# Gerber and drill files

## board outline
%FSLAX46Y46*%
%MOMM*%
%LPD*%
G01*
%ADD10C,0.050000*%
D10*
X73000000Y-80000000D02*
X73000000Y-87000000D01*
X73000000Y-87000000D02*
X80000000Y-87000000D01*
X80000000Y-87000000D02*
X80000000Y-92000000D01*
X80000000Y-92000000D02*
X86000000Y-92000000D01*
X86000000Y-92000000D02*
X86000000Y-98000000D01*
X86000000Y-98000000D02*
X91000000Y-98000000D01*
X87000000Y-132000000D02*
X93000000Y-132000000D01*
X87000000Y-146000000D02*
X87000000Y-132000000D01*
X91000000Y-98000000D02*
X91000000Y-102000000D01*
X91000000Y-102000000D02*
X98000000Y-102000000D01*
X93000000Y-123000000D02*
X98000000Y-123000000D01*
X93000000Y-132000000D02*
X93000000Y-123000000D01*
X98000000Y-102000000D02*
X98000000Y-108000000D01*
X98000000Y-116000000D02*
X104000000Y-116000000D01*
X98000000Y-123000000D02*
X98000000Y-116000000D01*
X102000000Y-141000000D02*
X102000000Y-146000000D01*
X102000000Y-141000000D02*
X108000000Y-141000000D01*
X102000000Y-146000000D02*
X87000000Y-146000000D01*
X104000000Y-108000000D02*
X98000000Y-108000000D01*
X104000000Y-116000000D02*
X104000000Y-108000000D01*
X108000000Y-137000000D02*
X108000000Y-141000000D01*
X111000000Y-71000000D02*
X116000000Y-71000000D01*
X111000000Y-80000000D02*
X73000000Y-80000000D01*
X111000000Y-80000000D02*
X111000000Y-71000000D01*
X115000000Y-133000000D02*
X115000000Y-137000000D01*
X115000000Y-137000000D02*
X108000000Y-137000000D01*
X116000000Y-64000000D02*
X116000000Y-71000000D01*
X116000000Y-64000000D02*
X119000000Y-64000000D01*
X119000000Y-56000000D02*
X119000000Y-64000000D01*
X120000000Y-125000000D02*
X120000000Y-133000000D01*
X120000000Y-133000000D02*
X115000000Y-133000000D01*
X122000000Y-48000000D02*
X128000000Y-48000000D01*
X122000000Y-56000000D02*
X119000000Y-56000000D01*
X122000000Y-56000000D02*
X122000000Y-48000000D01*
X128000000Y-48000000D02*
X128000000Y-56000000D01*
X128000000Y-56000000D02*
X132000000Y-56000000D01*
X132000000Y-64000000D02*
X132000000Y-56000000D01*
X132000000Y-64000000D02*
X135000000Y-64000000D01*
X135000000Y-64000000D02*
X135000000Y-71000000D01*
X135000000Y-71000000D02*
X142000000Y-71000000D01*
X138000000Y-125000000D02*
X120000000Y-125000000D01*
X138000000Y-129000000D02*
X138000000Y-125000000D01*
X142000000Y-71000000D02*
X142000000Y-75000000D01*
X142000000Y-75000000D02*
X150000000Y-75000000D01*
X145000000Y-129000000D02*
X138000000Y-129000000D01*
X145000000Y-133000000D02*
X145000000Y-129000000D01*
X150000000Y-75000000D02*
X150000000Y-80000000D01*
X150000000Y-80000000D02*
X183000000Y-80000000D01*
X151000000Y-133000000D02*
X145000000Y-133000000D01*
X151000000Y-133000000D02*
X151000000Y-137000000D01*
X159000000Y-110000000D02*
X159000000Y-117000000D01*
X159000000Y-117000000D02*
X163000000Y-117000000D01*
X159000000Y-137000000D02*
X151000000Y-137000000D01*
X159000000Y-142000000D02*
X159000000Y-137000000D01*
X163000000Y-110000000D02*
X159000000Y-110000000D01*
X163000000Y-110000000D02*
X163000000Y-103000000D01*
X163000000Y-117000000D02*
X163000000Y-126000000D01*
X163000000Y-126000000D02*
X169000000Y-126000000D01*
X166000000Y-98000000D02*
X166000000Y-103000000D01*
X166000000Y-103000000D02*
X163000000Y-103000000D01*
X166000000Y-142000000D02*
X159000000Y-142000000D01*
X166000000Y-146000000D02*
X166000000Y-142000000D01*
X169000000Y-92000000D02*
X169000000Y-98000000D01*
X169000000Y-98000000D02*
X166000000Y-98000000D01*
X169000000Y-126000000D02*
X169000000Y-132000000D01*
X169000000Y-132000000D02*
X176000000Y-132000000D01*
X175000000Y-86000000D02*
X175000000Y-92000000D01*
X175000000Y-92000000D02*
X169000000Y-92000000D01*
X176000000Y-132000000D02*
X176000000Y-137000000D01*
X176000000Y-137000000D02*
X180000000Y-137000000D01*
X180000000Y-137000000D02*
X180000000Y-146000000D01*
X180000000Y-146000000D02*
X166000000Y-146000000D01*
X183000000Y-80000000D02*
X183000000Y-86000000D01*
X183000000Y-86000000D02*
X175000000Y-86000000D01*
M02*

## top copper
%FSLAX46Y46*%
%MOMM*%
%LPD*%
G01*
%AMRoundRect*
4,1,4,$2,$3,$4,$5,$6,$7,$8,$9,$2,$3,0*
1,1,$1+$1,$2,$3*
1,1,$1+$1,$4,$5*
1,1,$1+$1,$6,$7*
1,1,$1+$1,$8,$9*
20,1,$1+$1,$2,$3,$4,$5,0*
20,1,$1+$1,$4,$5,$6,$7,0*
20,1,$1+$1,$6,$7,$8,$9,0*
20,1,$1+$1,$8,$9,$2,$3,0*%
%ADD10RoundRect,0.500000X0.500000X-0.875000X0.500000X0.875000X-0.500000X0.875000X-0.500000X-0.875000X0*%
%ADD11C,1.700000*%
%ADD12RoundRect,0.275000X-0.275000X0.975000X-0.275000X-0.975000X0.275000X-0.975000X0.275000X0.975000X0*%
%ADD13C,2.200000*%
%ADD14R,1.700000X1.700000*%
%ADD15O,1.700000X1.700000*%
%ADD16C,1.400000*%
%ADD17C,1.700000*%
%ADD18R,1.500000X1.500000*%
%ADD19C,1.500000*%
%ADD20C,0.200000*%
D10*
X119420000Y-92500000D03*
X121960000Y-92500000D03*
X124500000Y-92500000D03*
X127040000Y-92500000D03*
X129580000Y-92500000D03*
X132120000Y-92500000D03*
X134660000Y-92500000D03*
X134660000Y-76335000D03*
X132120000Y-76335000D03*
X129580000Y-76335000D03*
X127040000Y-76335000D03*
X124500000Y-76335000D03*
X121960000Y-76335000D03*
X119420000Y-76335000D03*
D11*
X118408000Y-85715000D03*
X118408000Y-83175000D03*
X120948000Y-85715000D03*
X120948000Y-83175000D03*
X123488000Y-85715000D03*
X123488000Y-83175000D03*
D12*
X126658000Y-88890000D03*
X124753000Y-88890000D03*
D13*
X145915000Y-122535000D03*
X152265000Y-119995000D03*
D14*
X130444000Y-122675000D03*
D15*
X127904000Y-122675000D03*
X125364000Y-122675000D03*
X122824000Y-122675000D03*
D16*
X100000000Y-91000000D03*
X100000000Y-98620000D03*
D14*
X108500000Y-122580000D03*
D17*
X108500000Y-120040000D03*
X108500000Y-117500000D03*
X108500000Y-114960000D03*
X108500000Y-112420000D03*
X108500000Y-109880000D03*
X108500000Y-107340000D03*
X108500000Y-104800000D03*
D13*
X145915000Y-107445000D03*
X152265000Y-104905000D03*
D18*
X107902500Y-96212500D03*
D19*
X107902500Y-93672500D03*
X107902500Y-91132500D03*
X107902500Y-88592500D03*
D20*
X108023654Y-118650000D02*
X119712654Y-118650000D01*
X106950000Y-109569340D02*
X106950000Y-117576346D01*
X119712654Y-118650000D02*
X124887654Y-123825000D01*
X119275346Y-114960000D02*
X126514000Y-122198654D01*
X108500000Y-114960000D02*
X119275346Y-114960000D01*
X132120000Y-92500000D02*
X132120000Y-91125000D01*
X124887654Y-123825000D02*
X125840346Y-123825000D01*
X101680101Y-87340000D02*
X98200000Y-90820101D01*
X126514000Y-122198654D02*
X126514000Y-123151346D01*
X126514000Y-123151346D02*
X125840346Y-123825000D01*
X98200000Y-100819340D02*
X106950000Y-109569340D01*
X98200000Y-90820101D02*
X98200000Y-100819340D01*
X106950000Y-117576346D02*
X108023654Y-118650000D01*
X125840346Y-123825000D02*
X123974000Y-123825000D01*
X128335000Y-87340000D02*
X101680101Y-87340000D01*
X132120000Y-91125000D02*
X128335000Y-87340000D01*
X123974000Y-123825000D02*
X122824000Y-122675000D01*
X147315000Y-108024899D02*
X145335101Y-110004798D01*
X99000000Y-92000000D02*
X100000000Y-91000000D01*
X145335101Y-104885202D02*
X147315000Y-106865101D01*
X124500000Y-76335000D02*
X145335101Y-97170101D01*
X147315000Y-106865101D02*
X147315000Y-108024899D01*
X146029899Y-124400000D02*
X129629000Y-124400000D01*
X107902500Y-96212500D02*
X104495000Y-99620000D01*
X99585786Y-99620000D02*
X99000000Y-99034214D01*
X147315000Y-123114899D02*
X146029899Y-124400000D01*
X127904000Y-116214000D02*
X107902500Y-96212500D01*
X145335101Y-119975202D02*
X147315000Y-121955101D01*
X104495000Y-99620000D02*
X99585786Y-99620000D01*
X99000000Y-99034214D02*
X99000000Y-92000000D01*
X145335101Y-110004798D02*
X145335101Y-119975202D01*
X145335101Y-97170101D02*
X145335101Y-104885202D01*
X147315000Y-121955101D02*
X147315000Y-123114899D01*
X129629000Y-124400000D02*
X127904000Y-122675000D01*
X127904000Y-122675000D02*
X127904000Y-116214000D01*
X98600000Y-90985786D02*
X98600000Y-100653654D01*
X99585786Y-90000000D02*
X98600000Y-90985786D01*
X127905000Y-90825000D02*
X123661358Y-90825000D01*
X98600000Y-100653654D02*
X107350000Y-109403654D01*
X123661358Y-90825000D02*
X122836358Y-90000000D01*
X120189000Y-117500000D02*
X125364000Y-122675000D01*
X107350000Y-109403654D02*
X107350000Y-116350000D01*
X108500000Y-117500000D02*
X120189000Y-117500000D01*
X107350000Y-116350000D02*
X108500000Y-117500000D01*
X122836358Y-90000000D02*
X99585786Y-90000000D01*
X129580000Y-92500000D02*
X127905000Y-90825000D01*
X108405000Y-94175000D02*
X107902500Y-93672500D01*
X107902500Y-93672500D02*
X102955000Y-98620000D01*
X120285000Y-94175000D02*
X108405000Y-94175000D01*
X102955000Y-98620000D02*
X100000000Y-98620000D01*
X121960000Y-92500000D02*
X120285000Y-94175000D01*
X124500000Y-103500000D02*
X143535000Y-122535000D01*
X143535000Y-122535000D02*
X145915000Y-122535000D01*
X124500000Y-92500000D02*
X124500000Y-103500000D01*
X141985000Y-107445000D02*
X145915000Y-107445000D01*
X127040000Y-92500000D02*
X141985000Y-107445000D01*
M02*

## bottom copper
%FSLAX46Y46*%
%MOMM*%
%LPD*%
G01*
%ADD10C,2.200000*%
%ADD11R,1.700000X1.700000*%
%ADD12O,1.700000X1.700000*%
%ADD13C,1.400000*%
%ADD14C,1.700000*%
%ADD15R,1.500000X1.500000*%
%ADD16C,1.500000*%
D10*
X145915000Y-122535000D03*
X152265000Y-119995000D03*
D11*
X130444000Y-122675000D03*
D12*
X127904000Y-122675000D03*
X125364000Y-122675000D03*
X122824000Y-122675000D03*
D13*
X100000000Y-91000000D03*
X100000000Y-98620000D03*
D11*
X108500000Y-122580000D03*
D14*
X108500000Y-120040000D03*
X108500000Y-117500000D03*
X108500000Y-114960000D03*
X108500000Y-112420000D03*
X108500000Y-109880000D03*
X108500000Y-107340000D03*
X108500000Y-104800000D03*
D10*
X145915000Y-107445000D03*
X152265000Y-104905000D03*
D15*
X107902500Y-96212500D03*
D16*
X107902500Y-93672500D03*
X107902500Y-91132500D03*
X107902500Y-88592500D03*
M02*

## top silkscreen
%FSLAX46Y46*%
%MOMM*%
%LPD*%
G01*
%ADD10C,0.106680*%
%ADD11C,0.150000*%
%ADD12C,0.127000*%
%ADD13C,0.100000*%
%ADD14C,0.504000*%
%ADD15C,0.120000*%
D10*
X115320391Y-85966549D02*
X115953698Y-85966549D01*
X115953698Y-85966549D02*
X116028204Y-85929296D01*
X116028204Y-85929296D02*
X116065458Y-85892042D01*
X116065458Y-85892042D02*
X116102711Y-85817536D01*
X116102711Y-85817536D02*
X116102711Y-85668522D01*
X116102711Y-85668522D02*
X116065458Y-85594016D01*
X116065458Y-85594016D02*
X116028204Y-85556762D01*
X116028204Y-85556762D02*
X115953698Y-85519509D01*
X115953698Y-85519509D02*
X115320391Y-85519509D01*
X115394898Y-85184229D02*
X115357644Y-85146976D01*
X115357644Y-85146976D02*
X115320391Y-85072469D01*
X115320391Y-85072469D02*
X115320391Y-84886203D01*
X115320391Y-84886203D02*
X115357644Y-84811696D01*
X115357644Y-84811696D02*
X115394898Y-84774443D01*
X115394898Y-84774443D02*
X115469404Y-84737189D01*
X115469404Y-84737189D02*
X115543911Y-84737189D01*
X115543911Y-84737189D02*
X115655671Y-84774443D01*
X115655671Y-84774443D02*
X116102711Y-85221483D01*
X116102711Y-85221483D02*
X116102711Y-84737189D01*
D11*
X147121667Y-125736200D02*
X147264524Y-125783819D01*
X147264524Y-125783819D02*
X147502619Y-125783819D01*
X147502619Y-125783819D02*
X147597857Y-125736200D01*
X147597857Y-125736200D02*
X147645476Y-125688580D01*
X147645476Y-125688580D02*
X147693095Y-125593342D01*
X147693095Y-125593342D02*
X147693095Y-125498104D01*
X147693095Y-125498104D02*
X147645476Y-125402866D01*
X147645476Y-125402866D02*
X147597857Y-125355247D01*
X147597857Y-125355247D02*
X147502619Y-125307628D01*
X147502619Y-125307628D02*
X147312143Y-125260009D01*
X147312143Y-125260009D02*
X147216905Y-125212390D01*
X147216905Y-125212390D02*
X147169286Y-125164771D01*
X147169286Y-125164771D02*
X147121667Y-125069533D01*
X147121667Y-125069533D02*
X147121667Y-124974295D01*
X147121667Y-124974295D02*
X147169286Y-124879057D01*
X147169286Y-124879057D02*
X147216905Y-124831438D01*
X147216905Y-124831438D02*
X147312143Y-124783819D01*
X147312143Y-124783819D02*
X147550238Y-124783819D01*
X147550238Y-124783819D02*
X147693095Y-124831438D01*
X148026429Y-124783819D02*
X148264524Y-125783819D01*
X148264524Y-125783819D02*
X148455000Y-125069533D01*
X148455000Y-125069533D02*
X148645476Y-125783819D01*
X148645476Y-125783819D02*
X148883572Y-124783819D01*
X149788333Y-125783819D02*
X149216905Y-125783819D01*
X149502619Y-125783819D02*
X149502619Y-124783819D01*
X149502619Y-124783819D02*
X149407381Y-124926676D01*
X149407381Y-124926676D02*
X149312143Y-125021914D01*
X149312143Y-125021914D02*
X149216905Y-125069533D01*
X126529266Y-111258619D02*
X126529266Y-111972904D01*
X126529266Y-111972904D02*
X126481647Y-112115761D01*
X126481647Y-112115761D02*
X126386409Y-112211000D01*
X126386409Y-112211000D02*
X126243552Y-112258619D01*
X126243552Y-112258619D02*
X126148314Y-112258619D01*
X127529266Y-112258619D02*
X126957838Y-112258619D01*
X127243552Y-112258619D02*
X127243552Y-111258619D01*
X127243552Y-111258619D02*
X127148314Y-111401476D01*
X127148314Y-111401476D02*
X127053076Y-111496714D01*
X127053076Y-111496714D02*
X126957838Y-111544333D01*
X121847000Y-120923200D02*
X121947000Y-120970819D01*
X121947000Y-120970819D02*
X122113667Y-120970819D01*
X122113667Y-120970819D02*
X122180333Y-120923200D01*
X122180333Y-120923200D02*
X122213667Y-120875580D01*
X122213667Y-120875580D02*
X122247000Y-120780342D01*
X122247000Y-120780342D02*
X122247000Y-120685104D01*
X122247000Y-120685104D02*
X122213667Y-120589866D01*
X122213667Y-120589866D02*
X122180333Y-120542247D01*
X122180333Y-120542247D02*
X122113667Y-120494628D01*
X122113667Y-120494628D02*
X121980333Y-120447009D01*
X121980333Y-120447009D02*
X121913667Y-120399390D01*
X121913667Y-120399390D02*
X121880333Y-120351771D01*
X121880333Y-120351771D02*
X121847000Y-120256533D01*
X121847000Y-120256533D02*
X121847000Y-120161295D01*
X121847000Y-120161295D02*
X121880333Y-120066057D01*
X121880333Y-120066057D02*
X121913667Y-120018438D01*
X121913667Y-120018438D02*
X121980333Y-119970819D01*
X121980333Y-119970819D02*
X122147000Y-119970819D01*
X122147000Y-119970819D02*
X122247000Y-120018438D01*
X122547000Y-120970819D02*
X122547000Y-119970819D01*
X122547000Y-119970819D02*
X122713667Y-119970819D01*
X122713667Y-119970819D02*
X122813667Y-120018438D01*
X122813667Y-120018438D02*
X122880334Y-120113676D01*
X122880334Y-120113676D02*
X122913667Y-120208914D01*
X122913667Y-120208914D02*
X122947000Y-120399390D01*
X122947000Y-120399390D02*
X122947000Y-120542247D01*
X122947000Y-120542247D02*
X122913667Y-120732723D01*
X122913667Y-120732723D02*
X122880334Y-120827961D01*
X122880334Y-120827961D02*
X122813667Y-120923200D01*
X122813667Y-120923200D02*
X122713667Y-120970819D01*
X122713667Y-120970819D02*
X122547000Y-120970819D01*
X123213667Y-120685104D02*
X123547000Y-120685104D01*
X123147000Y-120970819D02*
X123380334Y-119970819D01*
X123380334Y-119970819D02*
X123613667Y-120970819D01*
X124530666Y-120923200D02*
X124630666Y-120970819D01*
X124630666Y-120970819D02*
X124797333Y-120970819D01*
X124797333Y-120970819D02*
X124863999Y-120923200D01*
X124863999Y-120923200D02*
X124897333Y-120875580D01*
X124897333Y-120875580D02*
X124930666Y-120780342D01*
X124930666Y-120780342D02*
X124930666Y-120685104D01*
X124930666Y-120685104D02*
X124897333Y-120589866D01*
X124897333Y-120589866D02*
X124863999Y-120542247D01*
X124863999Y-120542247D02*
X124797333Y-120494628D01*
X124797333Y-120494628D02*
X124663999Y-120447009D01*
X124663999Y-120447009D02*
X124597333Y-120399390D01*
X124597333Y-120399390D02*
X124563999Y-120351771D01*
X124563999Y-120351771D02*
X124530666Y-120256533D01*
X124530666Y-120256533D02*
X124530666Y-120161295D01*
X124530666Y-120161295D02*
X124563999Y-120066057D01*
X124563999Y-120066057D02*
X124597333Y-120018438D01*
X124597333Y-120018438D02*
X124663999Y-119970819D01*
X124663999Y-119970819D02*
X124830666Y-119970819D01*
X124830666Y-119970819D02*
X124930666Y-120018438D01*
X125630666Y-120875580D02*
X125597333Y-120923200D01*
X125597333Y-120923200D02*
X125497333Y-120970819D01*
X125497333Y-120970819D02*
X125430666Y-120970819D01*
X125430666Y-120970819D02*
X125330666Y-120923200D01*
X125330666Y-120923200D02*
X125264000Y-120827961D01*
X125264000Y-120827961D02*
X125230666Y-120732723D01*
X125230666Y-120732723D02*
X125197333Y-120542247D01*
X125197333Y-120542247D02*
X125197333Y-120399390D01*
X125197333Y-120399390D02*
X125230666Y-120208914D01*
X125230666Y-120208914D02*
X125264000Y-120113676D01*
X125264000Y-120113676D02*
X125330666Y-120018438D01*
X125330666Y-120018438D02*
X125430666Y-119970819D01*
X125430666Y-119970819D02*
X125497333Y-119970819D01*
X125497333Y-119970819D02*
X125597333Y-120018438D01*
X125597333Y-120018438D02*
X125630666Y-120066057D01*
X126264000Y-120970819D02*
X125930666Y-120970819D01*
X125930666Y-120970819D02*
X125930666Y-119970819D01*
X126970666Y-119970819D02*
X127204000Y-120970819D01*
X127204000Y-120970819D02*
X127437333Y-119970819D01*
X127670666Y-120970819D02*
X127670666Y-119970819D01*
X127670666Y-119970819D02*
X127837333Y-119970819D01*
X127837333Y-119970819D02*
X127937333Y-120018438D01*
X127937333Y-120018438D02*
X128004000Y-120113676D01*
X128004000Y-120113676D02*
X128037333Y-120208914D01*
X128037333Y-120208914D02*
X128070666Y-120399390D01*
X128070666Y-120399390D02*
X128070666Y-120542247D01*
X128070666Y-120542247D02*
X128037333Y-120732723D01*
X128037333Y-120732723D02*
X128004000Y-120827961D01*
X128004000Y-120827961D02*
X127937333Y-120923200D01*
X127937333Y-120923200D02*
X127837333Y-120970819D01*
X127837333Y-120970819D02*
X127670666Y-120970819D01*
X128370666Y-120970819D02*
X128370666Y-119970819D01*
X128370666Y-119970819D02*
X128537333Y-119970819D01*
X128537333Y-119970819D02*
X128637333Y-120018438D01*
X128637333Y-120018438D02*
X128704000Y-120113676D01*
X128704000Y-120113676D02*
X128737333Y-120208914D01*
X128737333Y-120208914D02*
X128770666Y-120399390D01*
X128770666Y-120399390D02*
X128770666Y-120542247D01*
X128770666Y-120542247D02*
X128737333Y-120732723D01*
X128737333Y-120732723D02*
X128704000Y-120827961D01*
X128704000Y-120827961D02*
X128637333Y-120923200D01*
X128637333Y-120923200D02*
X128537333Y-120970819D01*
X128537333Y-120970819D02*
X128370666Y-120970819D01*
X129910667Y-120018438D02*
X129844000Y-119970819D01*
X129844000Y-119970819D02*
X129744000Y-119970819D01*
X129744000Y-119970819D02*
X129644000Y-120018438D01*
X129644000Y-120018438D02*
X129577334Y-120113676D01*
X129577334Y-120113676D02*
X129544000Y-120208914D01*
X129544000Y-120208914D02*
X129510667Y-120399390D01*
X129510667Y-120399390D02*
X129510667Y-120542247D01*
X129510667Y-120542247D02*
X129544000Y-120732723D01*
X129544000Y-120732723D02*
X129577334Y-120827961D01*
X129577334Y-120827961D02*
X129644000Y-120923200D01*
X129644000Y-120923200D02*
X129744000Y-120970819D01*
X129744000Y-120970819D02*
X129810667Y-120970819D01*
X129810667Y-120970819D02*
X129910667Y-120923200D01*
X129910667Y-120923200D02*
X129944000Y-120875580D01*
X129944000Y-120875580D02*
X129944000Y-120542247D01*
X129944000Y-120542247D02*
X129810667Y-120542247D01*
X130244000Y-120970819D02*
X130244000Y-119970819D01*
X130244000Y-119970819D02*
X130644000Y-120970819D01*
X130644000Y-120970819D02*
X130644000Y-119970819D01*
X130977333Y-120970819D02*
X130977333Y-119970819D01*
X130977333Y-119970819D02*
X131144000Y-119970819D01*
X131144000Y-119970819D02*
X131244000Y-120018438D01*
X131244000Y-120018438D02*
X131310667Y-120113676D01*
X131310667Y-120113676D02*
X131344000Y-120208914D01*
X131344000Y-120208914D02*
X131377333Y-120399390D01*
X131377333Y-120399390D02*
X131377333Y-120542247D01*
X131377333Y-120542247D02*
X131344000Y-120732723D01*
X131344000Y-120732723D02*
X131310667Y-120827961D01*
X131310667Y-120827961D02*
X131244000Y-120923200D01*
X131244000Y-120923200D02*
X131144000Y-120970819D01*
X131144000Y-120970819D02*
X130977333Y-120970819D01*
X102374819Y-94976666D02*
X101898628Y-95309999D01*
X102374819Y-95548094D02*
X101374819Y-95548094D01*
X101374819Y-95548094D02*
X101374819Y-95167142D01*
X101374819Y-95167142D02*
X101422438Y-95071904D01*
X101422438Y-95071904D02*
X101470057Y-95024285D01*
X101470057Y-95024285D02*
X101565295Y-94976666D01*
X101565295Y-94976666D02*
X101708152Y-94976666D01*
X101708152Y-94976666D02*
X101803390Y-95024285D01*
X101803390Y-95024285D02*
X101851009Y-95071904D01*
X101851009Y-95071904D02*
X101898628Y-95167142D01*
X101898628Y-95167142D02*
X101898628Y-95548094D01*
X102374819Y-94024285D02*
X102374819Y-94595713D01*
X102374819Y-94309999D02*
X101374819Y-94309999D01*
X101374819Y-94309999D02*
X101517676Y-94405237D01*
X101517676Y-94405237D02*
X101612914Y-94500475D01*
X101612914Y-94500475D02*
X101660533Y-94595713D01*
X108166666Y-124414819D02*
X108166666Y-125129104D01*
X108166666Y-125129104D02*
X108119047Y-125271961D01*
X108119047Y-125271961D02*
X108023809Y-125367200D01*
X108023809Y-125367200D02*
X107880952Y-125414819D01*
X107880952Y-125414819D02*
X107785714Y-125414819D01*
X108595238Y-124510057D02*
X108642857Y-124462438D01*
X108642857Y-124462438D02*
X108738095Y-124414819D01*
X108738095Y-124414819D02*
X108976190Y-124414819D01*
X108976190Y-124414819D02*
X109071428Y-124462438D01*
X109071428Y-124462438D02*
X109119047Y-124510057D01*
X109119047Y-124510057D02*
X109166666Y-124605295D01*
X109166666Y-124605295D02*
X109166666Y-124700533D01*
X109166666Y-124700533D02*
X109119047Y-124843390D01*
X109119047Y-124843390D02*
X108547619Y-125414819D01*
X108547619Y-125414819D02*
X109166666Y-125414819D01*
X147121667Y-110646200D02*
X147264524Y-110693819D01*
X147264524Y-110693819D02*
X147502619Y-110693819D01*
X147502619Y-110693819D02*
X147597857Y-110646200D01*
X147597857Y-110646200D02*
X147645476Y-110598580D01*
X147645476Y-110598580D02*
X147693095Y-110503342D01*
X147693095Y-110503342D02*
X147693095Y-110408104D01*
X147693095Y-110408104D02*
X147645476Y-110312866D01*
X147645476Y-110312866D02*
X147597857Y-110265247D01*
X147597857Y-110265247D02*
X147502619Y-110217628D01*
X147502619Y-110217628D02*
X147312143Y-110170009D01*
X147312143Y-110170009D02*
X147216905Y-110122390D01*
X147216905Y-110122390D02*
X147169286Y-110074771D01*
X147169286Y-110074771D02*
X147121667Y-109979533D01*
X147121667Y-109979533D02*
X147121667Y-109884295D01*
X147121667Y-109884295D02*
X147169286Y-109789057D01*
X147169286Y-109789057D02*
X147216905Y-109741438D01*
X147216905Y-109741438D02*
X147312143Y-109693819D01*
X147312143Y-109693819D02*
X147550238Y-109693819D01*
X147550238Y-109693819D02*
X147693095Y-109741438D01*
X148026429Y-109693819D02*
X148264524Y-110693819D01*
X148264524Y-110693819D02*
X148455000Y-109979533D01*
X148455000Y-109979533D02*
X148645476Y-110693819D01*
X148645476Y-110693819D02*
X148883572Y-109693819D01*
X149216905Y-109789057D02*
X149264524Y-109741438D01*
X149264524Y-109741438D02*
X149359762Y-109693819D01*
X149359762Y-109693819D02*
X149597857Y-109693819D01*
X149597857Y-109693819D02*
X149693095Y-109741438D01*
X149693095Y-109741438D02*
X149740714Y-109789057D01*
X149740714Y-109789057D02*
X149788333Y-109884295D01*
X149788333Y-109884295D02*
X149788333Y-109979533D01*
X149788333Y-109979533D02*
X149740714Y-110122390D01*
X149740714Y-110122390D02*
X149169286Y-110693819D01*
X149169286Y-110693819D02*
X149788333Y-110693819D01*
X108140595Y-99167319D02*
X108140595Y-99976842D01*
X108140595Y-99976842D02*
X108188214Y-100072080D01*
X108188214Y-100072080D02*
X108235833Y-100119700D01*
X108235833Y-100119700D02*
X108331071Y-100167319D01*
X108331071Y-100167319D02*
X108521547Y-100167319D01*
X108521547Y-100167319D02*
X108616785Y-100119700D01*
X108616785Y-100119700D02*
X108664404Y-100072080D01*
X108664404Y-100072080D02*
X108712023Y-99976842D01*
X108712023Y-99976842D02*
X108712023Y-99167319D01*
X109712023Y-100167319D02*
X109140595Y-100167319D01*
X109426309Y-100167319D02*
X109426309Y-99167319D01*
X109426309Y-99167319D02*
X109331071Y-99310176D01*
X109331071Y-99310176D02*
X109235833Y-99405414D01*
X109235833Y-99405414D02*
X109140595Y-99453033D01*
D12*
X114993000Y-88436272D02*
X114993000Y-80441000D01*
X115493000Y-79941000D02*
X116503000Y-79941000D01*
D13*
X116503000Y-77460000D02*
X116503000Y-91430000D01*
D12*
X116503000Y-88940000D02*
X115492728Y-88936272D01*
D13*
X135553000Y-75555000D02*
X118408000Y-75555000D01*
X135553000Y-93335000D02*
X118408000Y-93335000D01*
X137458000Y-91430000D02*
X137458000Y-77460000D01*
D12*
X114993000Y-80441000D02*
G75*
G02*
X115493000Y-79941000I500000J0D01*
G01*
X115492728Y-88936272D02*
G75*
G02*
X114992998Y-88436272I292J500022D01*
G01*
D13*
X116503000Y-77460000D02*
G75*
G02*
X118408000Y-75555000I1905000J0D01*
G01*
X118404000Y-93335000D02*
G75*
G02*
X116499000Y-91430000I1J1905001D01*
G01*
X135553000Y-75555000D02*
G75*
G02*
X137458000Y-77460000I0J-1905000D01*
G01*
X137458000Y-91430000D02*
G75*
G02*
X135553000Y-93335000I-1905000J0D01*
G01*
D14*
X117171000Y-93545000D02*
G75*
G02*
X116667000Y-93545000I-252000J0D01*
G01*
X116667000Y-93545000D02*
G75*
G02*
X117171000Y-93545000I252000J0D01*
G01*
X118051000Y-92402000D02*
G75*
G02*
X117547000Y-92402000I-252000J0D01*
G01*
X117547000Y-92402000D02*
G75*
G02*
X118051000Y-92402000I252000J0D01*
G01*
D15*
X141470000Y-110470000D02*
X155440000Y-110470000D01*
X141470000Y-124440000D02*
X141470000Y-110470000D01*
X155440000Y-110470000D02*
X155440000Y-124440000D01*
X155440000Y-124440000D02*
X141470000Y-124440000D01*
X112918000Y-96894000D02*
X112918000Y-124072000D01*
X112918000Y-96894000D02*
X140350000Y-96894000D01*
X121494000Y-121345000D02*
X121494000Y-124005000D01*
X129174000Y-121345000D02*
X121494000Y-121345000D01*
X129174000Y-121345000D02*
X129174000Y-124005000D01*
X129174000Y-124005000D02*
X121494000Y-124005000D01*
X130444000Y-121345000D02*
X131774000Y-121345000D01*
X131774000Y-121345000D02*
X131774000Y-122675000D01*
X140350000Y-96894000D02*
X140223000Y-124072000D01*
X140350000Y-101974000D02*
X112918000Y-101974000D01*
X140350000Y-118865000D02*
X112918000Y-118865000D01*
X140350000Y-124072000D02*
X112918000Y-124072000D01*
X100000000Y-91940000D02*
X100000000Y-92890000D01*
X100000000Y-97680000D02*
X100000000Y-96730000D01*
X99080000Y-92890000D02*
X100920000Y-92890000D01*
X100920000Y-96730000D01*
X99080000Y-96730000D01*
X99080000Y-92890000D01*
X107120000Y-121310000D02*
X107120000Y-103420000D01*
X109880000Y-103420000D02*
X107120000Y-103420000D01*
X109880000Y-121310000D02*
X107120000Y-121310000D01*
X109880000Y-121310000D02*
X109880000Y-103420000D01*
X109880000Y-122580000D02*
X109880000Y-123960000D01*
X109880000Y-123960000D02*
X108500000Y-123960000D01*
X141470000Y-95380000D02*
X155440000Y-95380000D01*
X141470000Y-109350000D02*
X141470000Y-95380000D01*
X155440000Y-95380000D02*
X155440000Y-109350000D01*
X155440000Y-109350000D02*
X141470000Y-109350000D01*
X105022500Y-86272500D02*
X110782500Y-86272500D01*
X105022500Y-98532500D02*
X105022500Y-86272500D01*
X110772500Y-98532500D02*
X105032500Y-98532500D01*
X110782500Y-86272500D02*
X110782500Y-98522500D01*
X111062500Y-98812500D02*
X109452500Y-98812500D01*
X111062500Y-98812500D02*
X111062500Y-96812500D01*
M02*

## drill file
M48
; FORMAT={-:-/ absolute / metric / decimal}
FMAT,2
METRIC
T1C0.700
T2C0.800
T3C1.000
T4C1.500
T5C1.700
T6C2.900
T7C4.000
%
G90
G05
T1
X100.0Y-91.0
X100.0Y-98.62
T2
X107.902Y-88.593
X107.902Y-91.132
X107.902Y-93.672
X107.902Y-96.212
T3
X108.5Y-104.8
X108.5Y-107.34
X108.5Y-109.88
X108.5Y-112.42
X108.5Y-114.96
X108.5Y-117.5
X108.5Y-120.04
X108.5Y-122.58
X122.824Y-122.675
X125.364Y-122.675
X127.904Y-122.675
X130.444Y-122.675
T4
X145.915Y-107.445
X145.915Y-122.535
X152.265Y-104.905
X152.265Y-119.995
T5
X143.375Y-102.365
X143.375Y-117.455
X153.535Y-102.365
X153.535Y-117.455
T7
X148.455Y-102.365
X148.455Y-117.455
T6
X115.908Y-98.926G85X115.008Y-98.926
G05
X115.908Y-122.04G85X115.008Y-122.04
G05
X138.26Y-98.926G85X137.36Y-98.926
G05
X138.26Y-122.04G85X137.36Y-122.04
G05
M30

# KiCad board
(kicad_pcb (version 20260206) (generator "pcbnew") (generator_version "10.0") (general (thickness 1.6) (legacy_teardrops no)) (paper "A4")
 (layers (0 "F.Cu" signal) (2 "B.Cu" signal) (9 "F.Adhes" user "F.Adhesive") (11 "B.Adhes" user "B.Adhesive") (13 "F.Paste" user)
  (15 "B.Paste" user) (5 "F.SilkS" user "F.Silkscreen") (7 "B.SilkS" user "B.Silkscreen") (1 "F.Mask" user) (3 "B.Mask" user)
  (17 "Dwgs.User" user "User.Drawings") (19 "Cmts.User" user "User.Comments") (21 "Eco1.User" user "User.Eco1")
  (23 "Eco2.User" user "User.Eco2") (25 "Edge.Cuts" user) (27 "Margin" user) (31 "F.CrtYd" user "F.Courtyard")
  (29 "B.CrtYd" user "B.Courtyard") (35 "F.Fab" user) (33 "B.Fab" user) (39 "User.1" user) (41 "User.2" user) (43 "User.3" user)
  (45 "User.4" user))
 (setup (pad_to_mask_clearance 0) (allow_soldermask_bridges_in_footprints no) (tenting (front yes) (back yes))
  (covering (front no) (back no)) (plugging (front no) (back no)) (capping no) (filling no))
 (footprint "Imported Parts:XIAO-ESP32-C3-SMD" (layer "F.Cu") (at 137.54 93.335 90)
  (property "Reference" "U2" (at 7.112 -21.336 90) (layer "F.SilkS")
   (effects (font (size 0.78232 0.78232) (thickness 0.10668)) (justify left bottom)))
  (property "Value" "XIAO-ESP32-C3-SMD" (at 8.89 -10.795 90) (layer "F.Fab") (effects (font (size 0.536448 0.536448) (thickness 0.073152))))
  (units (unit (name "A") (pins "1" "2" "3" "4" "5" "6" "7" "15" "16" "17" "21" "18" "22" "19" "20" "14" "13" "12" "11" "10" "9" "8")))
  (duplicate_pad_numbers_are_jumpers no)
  (fp_line (start 4.898728 -22.547) (end 12.894 -22.547) (stroke (width 0.127) (type solid)) (layer "F.SilkS"))
  (fp_line (start 13.394 -22.047) (end 13.394 -21.037) (stroke (width 0.127) (type solid)) (layer "F.SilkS"))
  (fp_line (start 15.875 -21.037) (end 1.905 -21.037) (stroke (width 0.1) (type solid)) (layer "F.SilkS"))
  (fp_line (start 4.395 -21.037) (end 4.398728 -22.047272) (stroke (width 0.127) (type solid)) (layer "F.SilkS"))
  (fp_line (start 17.78 -1.987) (end 17.78 -19.132) (stroke (width 0.1) (type solid)) (layer "F.SilkS"))
  (fp_line (start 0 -1.987) (end 0 -19.132) (stroke (width 0.1) (type solid)) (layer "F.SilkS"))
  (fp_line (start 1.905 -0.082) (end 15.875 -0.082) (stroke (width 0.1) (type solid)) (layer "F.SilkS"))
  (fp_arc (start 12.894 -22.547) (mid 13.247553 -22.400553) (end 13.394 -22.047) (stroke (width 0.127) (type default)) (layer "F.SilkS"))
  (fp_arc (start 4.398728 -22.047272) (mid 4.545272 -22.40064) (end 4.898728 -22.547) (stroke (width 0.127) (type default))
   (layer "F.SilkS"))
  (fp_arc (start 15.875 -21.037) (mid 17.222038 -20.479038) (end 17.78 -19.132) (stroke (width 0.1) (type solid)) (layer "F.SilkS"))
  (fp_arc (start 0 -19.136) (mid 0.557962 -20.483038) (end 1.905 -21.041) (stroke (width 0.1) (type solid)) (layer "F.SilkS"))
  (fp_arc (start 17.78 -1.987) (mid 17.222038 -0.639962) (end 15.875 -0.082) (stroke (width 0.1) (type solid)) (layer "F.SilkS"))
  (fp_arc (start 1.905 -0.082) (mid 0.557962 -0.639962) (end 0 -1.987) (stroke (width 0.1) (type solid)) (layer "F.SilkS"))
  (fp_circle (center -0.21 -20.621) (end -0.21 -20.875) (stroke (width 0.5) (type solid)) (fill yes) (layer "F.SilkS"))
  (fp_circle (center 0.933 -19.741) (end 0.933 -19.995) (stroke (width 0.5) (type solid)) (fill yes) (layer "F.SilkS"))
  (pad "1" smd roundrect (at 0.835 -18.12 90) (size 2.75 2) (layers "F.Cu" "F.Mask" "F.Paste") (roundrect_rratio 0.25)
   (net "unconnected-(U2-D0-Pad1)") (solder_mask_margin 0.0508) (thermal_bridge_angle 45))
  (pad "2" smd roundrect (at 0.835 -15.58 90) (size 2.75 2) (layers "F.Cu" "F.Mask" "F.Paste") (roundrect_rratio 0.25) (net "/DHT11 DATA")
   (solder_mask_margin 0.0508) (thermal_bridge_angle 45))
  (pad "3" smd roundrect (at 0.835 -13.04 90) (size 2.75 2) (layers "F.Cu" "F.Mask" "F.Paste") (roundrect_rratio 0.25) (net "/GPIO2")
   (solder_mask_margin 0.0508) (thermal_bridge_angle 45))
  (pad "4" smd roundrect (at 0.835 -10.5 90) (size 2.75 2) (layers "F.Cu" "F.Mask" "F.Paste") (roundrect_rratio 0.25) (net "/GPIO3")
   (solder_mask_margin 0.0508) (thermal_bridge_angle 45))
  (pad "5" smd roundrect (at 0.835 -7.96 90) (size 2.75 2) (layers "F.Cu" "F.Mask" "F.Paste") (roundrect_rratio 0.25) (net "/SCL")
   (solder_mask_margin 0.0508) (thermal_bridge_angle 45))
  (pad "6" smd roundrect (at 0.835 -5.42 90) (size 2.75 2) (layers "F.Cu" "F.Mask" "F.Paste") (roundrect_rratio 0.25) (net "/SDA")
   (solder_mask_margin 0.0508) (thermal_bridge_angle 45))
  (pad "7" smd roundrect (at 0.835 -2.88 90) (size 2.75 2) (layers "F.Cu" "F.Mask" "F.Paste") (roundrect_rratio 0.25)
   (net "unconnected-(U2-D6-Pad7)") (solder_mask_margin 0.0508) (thermal_bridge_angle 45))
  (pad "8" smd roundrect (at 17 -2.88 90) (size 2.75 2) (layers "F.Cu" "F.Mask" "F.Paste") (roundrect_rratio 0.25)
   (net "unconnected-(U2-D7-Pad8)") (solder_mask_margin 0.0508) (thermal_bridge_angle 45))
  (pad "9" smd roundrect (at 17 -5.42 90) (size 2.75 2) (layers "F.Cu" "F.Mask" "F.Paste") (roundrect_rratio 0.25)
   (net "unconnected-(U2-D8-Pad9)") (solder_mask_margin 0.0508) (thermal_bridge_angle 45))
  (pad "10" smd roundrect (at 17 -7.96 90) (size 2.75 2) (layers "F.Cu" "F.Mask" "F.Paste") (roundrect_rratio 0.25)
   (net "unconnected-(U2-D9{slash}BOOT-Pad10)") (solder_mask_margin 0.0508) (thermal_bridge_angle 45))
  (pad "11" smd roundrect (at 17 -10.5 90) (size 2.75 2) (layers "F.Cu" "F.Mask" "F.Paste") (roundrect_rratio 0.25)
   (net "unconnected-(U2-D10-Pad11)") (solder_mask_margin 0.0508) (thermal_bridge_angle 45))
  (pad "12" smd roundrect (at 17 -13.04 90) (size 2.75 2) (layers "F.Cu" "F.Mask" "F.Paste") (roundrect_rratio 0.25) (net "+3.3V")
   (solder_mask_margin 0.0508) (thermal_bridge_angle 45))
  (pad "13" smd roundrect (at 17 -15.58 90) (size 2.75 2) (layers "F.Cu" "F.Mask" "F.Paste") (roundrect_rratio 0.25) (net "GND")
   (solder_mask_margin 0.0508) (thermal_bridge_angle 45))
  (pad "14" smd roundrect (at 17 -18.12 90) (size 2.75 2) (layers "F.Cu" "F.Mask" "F.Paste") (roundrect_rratio 0.25) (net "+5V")
   (solder_mask_margin 0.0508) (thermal_bridge_angle 45))
  (pad "15" smd circle (at 7.62 -19.132 90) (size 1.7 1.7) (layers "F.Cu" "F.Mask" "F.Paste") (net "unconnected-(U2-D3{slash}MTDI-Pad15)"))
  (pad "16" smd circle (at 10.16 -19.132 90) (size 1.7 1.7) (layers "F.Cu" "F.Mask" "F.Paste") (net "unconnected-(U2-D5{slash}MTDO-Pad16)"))
  (pad "17" smd circle (at 7.62 -16.592 90) (size 1.7 1.7) (layers "F.Cu" "F.Mask" "F.Paste") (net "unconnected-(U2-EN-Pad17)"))
  (pad "18" smd circle (at 10.16 -16.592 90) (size 1.7 1.7) (layers "F.Cu" "F.Mask" "F.Paste") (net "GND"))
  (pad "19" smd circle (at 7.62 -14.052 90) (size 1.7 1.7) (layers "F.Cu" "F.Mask" "F.Paste") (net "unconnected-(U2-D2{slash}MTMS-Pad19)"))
  (pad "20" smd circle (at 10.16 -14.052 90) (size 1.7 1.7) (layers "F.Cu" "F.Mask" "F.Paste") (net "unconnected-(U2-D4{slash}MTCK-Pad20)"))
  (pad "21" smd roundrect (at 4.445 -10.882 270) (size 2.5 1.1) (layers "F.Cu" "F.Mask" "F.Paste") (roundrect_rratio 0.25)
   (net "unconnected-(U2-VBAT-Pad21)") (thermal_bridge_angle 45))
  (pad "22" smd roundrect (at 4.445 -12.787 270) (size 2.5 1.1) (layers "F.Cu" "F.Mask" "F.Paste") (roundrect_rratio 0.25)
   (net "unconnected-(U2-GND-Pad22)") (thermal_bridge_angle 45)))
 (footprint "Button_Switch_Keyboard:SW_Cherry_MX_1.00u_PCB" (layer "F.Cu") (at 145.915 122.535 180)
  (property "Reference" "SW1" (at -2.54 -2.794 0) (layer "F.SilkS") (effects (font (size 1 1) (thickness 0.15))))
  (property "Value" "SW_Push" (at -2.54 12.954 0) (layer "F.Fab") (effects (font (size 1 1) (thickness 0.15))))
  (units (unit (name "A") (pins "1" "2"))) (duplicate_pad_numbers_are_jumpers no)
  (fp_line (start 4.445 12.065) (end -9.525 12.065) (stroke (width 0.12) (type solid)) (layer "F.SilkS"))
  (fp_line (start 4.445 -1.905) (end 4.445 12.065) (stroke (width 0.12) (type solid)) (layer "F.SilkS"))
  (fp_line (start -9.525 12.065) (end -9.525 -1.905) (stroke (width 0.12) (type solid)) (layer "F.SilkS"))
  (fp_line (start -9.525 -1.905) (end 4.445 -1.905) (stroke (width 0.12) (type solid)) (layer "F.SilkS"))
  (pad "" np_thru_hole circle (at -7.62 5.08 180) (size 1.7 1.7) (drill 1.7) (layers "*.Cu" "*.Mask"))
  (pad "" np_thru_hole circle (at -2.54 5.08 180) (size 4 4) (drill 4) (layers "*.Cu" "*.Mask"))
  (pad "" np_thru_hole circle (at 2.54 5.08 180) (size 1.7 1.7) (drill 1.7) (layers "*.Cu" "*.Mask"))
  (pad "1" thru_hole circle (at 0 0 180) (size 2.2 2.2) (drill 1.5) (layers "*.Cu" "*.Mask") (remove_unused_layers no) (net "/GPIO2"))
  (pad "2" thru_hole circle (at -6.35 2.54 180) (size 2.2 2.2) (drill 1.5) (layers "*.Cu" "*.Mask") (remove_unused_layers no) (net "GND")))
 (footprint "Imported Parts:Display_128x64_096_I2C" (layer "F.Cu") (at 126.634 122.675 180)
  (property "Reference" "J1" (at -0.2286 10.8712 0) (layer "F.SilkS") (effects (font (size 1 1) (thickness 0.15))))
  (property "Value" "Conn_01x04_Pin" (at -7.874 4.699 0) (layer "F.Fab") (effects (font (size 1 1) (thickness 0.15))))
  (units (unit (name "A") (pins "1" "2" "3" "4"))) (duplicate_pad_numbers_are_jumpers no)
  (fp_line (start 13.716 25.781) (end 13.716 -1.397) (stroke (width 0.12) (type solid)) (layer "F.SilkS"))
  (fp_line (start 13.716 25.781) (end -13.716 25.781) (stroke (width 0.12) (type solid)) (layer "F.SilkS"))
  (fp_line (start 5.14 1.33) (end 5.14 -1.33) (stroke (width 0.12) (type solid)) (layer "F.SilkS"))
  (fp_line (start -2.54 1.33) (end 5.14 1.33) (stroke (width 0.12) (type solid)) (layer "F.SilkS"))
  (fp_line (start -2.54 1.33) (end -2.54 -1.33) (stroke (width 0.12) (type solid)) (layer "F.SilkS"))
  (fp_line (start -2.54 -1.33) (end 5.14 -1.33) (stroke (width 0.12) (type solid)) (layer "F.SilkS"))
  (fp_line (start -3.81 1.33) (end -5.14 1.33) (stroke (width 0.12) (type solid)) (layer "F.SilkS"))
  (fp_line (start -5.14 1.33) (end -5.14 0) (stroke (width 0.12) (type solid)) (layer "F.SilkS"))
  (fp_line (start -13.716 25.781) (end -13.589 -1.397) (stroke (width 0.12) (type solid)) (layer "F.SilkS"))
  (fp_line (start -13.716 20.701) (end 13.716 20.701) (stroke (width 0.12) (type solid)) (layer "F.SilkS"))
  (fp_line (start -13.716 3.81) (end 13.716 3.81) (stroke (width 0.12) (type solid)) (layer "F.SilkS"))
  (fp_line (start -13.716 -1.397) (end 13.716 -1.397) (stroke (width 0.12) (type solid)) (layer "F.SilkS"))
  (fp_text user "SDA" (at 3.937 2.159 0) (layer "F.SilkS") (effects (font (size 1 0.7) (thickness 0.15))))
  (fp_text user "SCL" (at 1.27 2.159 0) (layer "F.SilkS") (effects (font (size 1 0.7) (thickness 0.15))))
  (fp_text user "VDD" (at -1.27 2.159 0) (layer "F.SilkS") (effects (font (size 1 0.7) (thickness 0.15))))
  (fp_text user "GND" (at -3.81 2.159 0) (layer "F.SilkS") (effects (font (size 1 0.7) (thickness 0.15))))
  (pad "" np_thru_hole oval (at -11.176 0.635 180) (size 3.8 2.9) (drill oval 3.8 2.9) (layers "*.Cu" "*.Mask"))
  (pad "" np_thru_hole oval (at -11.176 23.749 180) (size 3.8 2.9) (drill oval 3.8 2.9) (layers "*.Cu" "*.Mask"))
  (pad "" np_thru_hole oval (at 11.176 0.635 180) (size 3.8 2.9) (drill oval 3.8 2.9) (layers "*.Cu" "*.Mask"))
  (pad "" np_thru_hole oval (at 11.176 23.749 180) (size 3.8 2.9) (drill oval 3.8 2.9) (layers "*.Cu" "*.Mask"))
  (pad "1" thru_hole rect (at -3.81 0 270) (size 1.7 1.7) (drill 1) (layers "*.Cu" "*.Mask") (remove_unused_layers no) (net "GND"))
  (pad "2" thru_hole oval (at -1.27 0 270) (size 1.7 1.7) (drill 1) (layers "*.Cu" "*.Mask") (remove_unused_layers no) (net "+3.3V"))
  (pad "3" thru_hole oval (at 1.27 0 270) (size 1.7 1.7) (drill 1) (layers "*.Cu" "*.Mask") (remove_unused_layers no) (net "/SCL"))
  (pad "4" thru_hole oval (at 3.81 0 270) (size 1.7 1.7) (drill 1) (layers "*.Cu" "*.Mask") (remove_unused_layers no) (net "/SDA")))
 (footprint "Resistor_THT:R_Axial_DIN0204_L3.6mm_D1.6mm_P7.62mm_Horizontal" (layer "F.Cu") (at 100 91 -90)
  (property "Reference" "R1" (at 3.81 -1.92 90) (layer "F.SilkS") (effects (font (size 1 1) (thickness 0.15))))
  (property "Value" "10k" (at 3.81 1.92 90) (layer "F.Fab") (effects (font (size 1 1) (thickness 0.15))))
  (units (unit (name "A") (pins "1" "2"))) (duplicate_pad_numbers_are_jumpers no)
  (fp_line (start 0.94 0) (end 1.89 0) (stroke (width 0.12) (type solid)) (layer "F.SilkS"))
  (fp_line (start 6.68 0) (end 5.73 0) (stroke (width 0.12) (type solid)) (layer "F.SilkS"))
  (fp_rect (start 1.89 -0.92) (end 5.73 0.92) (stroke (width 0.12) (type solid)) (fill no) (layer "F.SilkS"))
  (pad "1" thru_hole circle (at 0 0 270) (size 1.4 1.4) (drill 0.7) (layers "*.Cu" "*.Mask") (remove_unused_layers no) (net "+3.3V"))
  (pad "2" thru_hole circle (at 7.62 0 270) (size 1.4 1.4) (drill 0.7) (layers "*.Cu" "*.Mask") (remove_unused_layers no)
   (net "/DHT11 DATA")))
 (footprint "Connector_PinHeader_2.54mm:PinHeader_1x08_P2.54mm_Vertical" (layer "F.Cu") (at 108.5 122.58 180)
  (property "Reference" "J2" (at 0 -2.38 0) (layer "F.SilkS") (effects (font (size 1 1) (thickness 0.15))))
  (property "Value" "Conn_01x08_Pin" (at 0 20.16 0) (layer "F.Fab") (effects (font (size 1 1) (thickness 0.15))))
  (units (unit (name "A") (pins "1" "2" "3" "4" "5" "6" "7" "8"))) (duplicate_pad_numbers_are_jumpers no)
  (fp_line (start 1.38 1.27) (end 1.38 19.16) (stroke (width 0.12) (type solid)) (layer "F.SilkS"))
  (fp_line (start -1.38 19.16) (end 1.38 19.16) (stroke (width 0.12) (type solid)) (layer "F.SilkS"))
  (fp_line (start -1.38 1.27) (end 1.38 1.27) (stroke (width 0.12) (type solid)) (layer "F.SilkS"))
  (fp_line (start -1.38 1.27) (end -1.38 19.16) (stroke (width 0.12) (type solid)) (layer "F.SilkS"))
  (fp_line (start -1.38 0) (end -1.38 -1.38) (stroke (width 0.12) (type solid)) (layer "F.SilkS"))
  (fp_line (start -1.38 -1.38) (end 0 -1.38) (stroke (width 0.12) (type solid)) (layer "F.SilkS"))
  (pad "1" thru_hole rect (at 0 0 180) (size 1.7 1.7) (drill 1) (layers "*.Cu" "*.Mask") (remove_unused_layers no) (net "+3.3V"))
  (pad "2" thru_hole circle (at 0 2.54 180) (size 1.7 1.7) (drill 1) (layers "*.Cu" "*.Mask") (remove_unused_layers no) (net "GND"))
  (pad "3" thru_hole circle (at 0 5.08 180) (size 1.7 1.7) (drill 1) (layers "*.Cu" "*.Mask") (remove_unused_layers no) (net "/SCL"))
  (pad "4" thru_hole circle (at 0 7.62 180) (size 1.7 1.7) (drill 1) (layers "*.Cu" "*.Mask") (remove_unused_layers no) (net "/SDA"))
  (pad "5" thru_hole circle (at 0 10.16 180) (size 1.7 1.7) (drill 1) (layers "*.Cu" "*.Mask") (remove_unused_layers no)
   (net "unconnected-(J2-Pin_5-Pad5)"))
  (pad "6" thru_hole circle (at 0 12.7 180) (size 1.7 1.7) (drill 1) (layers "*.Cu" "*.Mask") (remove_unused_layers no)
   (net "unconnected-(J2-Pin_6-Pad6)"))
  (pad "7" thru_hole circle (at 0 15.24 180) (size 1.7 1.7) (drill 1) (layers "*.Cu" "*.Mask") (remove_unused_layers no)
   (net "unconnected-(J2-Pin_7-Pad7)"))
  (pad "8" thru_hole circle (at 0 17.78 180) (size 1.7 1.7) (drill 1) (layers "*.Cu" "*.Mask") (remove_unused_layers no)
   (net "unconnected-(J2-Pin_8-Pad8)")))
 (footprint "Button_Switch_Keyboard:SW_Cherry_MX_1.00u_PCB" (layer "F.Cu") (at 145.915 107.445 180)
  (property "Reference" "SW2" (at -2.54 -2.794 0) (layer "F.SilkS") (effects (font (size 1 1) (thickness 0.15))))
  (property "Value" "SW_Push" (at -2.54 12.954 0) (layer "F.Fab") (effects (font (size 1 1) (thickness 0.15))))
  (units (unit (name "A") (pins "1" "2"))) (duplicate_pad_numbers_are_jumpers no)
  (fp_line (start 4.445 12.065) (end -9.525 12.065) (stroke (width 0.12) (type solid)) (layer "F.SilkS"))
  (fp_line (start 4.445 -1.905) (end 4.445 12.065) (stroke (width 0.12) (type solid)) (layer "F.SilkS"))
  (fp_line (start -9.525 12.065) (end -9.525 -1.905) (stroke (width 0.12) (type solid)) (layer "F.SilkS"))
  (fp_line (start -9.525 -1.905) (end 4.445 -1.905) (stroke (width 0.12) (type solid)) (layer "F.SilkS"))
  (pad "" np_thru_hole circle (at -7.62 5.08 180) (size 1.7 1.7) (drill 1.7) (layers "*.Cu" "*.Mask"))
  (pad "" np_thru_hole circle (at -2.54 5.08 180) (size 4 4) (drill 4) (layers "*.Cu" "*.Mask"))
  (pad "" np_thru_hole circle (at 2.54 5.08 180) (size 1.7 1.7) (drill 1.7) (layers "*.Cu" "*.Mask"))
  (pad "1" thru_hole circle (at 0 0 180) (size 2.2 2.2) (drill 1.5) (layers "*.Cu" "*.Mask") (remove_unused_layers no) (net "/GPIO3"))
  (pad "2" thru_hole circle (at -6.35 2.54 180) (size 2.2 2.2) (drill 1.5) (layers "*.Cu" "*.Mask") (remove_unused_layers no) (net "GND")))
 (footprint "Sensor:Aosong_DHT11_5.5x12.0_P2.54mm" (layer "F.Cu") (at 107.9025 96.2125 180)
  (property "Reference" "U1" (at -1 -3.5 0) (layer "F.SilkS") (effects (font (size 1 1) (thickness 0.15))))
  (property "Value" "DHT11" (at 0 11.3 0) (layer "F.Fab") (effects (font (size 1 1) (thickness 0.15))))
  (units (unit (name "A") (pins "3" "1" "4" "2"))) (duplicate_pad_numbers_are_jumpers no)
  (fp_line (start 2.88 9.94) (end -2.88 9.94) (stroke (width 0.12) (type solid)) (layer "F.SilkS"))
  (fp_line (start 2.88 -2.32) (end 2.88 9.94) (stroke (width 0.12) (type solid)) (layer "F.SilkS"))
  (fp_line (start -2.87 -2.32) (end 2.87 -2.32) (stroke (width 0.12) (type solid)) (layer "F.SilkS"))
  (fp_line (start -2.88 9.94) (end -2.88 -2.31) (stroke (width 0.12) (type solid)) (layer "F.SilkS"))
  (fp_line (start -3.16 -2.6) (end -1.55 -2.6) (stroke (width 0.12) (type solid)) (layer "F.SilkS"))
  (fp_line (start -3.16 -2.6) (end -3.16 -0.6) (stroke (width 0.12) (type solid)) (layer "F.SilkS"))
  (pad "1" thru_hole rect (at 0 0 180) (size 1.5 1.5) (drill 0.8) (layers "*.Cu" "*.Mask") (remove_unused_layers no) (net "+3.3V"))
  (pad "2" thru_hole circle (at 0 2.54 180) (size 1.5 1.5) (drill 0.8) (layers "*.Cu" "*.Mask") (remove_unused_layers no)
   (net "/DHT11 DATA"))
  (pad "3" thru_hole circle (at 0 5.08 180) (size 1.5 1.5) (drill 0.8) (layers "*.Cu" "*.Mask") (remove_unused_layers no)
   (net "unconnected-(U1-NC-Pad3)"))
  (pad "4" thru_hole circle (at 0 7.62 180) (size 1.5 1.5) (drill 0.8) (layers "*.Cu" "*.Mask") (remove_unused_layers no) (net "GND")))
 (gr_line (start 73 80) (end 73 87) (stroke (width 0.05) (type default)) (layer "Edge.Cuts"))
 (gr_line (start 73 87) (end 80 87) (stroke (width 0.05) (type default)) (layer "Edge.Cuts"))
 (gr_line (start 80 87) (end 80 92) (stroke (width 0.05) (type default)) (layer "Edge.Cuts"))
 (gr_line (start 80 92) (end 86 92) (stroke (width 0.05) (type default)) (layer "Edge.Cuts"))
 (gr_line (start 86 92) (end 86 98) (stroke (width 0.05) (type default)) (layer "Edge.Cuts"))
 (gr_line (start 86 98) (end 91 98) (stroke (width 0.05) (type default)) (layer "Edge.Cuts"))
 (gr_line (start 87 132) (end 93 132) (stroke (width 0.05) (type default)) (layer "Edge.Cuts"))
 (gr_line (start 87 146) (end 87 132) (stroke (width 0.05) (type default)) (layer "Edge.Cuts"))
 (gr_line (start 91 98) (end 91 102) (stroke (width 0.05) (type default)) (layer "Edge.Cuts"))
 (gr_line (start 91 102) (end 98 102) (stroke (width 0.05) (type default)) (layer "Edge.Cuts"))
 (gr_line (start 93 123) (end 98 123) (stroke (width 0.05) (type default)) (layer "Edge.Cuts"))
 (gr_line (start 93 132) (end 93 123) (stroke (width 0.05) (type default)) (layer "Edge.Cuts"))
 (gr_line (start 98 102) (end 98 108) (stroke (width 0.05) (type default)) (layer "Edge.Cuts"))
 (gr_line (start 98 116) (end 104 116) (stroke (width 0.05) (type default)) (layer "Edge.Cuts"))
 (gr_line (start 98 123) (end 98 116) (stroke (width 0.05) (type default)) (layer "Edge.Cuts"))
 (gr_line (start 102 141) (end 102 146) (stroke (width 0.05) (type default)) (layer "Edge.Cuts"))
 (gr_line (start 102 141) (end 108 141) (stroke (width 0.05) (type default)) (layer "Edge.Cuts"))
 (gr_line (start 102 146) (end 87 146) (stroke (width 0.05) (type default)) (layer "Edge.Cuts"))
 (gr_line (start 104 108) (end 98 108) (stroke (width 0.05) (type default)) (layer "Edge.Cuts"))
 (gr_line (start 104 116) (end 104 108) (stroke (width 0.05) (type default)) (layer "Edge.Cuts"))
 (gr_line (start 108 137) (end 108 141) (stroke (width 0.05) (type default)) (layer "Edge.Cuts"))
 (gr_line (start 111 71) (end 116 71) (stroke (width 0.05) (type default)) (layer "Edge.Cuts"))
 (gr_line (start 111 80) (end 73 80) (stroke (width 0.05) (type default)) (layer "Edge.Cuts"))
 (gr_line (start 111 80) (end 111 71) (stroke (width 0.05) (type default)) (layer "Edge.Cuts"))
 (gr_line (start 115 133) (end 115 137) (stroke (width 0.05) (type default)) (layer "Edge.Cuts"))
 (gr_line (start 115 137) (end 108 137) (stroke (width 0.05) (type default)) (layer "Edge.Cuts"))
 (gr_line (start 116 64) (end 116 71) (stroke (width 0.05) (type default)) (layer "Edge.Cuts"))
 (gr_line (start 116 64) (end 119 64) (stroke (width 0.05) (type default)) (layer "Edge.Cuts"))
 (gr_line (start 119 56) (end 119 64) (stroke (width 0.05) (type default)) (layer "Edge.Cuts"))
 (gr_line (start 120 125) (end 120 133) (stroke (width 0.05) (type default)) (layer "Edge.Cuts"))
 (gr_line (start 120 133) (end 115 133) (stroke (width 0.05) (type default)) (layer "Edge.Cuts"))
 (gr_line (start 122 48) (end 128 48) (stroke (width 0.05) (type default)) (layer "Edge.Cuts"))
 (gr_line (start 122 56) (end 119 56) (stroke (width 0.05) (type default)) (layer "Edge.Cuts"))
 (gr_line (start 122 56) (end 122 48) (stroke (width 0.05) (type default)) (layer "Edge.Cuts"))
 (gr_line (start 128 48) (end 128 56) (stroke (width 0.05) (type default)) (layer "Edge.Cuts"))
 (gr_line (start 128 56) (end 132 56) (stroke (width 0.05) (type default)) (layer "Edge.Cuts"))
 (gr_line (start 132 64) (end 132 56) (stroke (width 0.05) (type default)) (layer "Edge.Cuts"))
 (gr_line (start 132 64) (end 135 64) (stroke (width 0.05) (type default)) (layer "Edge.Cuts"))
 (gr_line (start 135 64) (end 135 71) (stroke (width 0.05) (type default)) (layer "Edge.Cuts"))
 (gr_line (start 135 71) (end 142 71) (stroke (width 0.05) (type default)) (layer "Edge.Cuts"))
 (gr_line (start 138 125) (end 120 125) (stroke (width 0.05) (type default)) (layer "Edge.Cuts"))
 (gr_line (start 138 129) (end 138 125) (stroke (width 0.05) (type default)) (layer "Edge.Cuts"))
 (gr_line (start 142 71) (end 142 75) (stroke (width 0.05) (type default)) (layer "Edge.Cuts"))
 (gr_line (start 142 75) (end 150 75) (stroke (width 0.05) (type default)) (layer "Edge.Cuts"))
 (gr_line (start 145 129) (end 138 129) (stroke (width 0.05) (type default)) (layer "Edge.Cuts"))
 (gr_line (start 145 133) (end 145 129) (stroke (width 0.05) (type default)) (layer "Edge.Cuts"))
 (gr_line (start 150 75) (end 150 80) (stroke (width 0.05) (type default)) (layer "Edge.Cuts"))
 (gr_line (start 150 80) (end 183 80) (stroke (width 0.05) (type default)) (layer "Edge.Cuts"))
 (gr_line (start 151 133) (end 145 133) (stroke (width 0.05) (type default)) (layer "Edge.Cuts"))
 (gr_line (start 151 133) (end 151 137) (stroke (width 0.05) (type default)) (layer "Edge.Cuts"))
 (gr_line (start 159 110) (end 159 117) (stroke (width 0.05) (type default)) (layer "Edge.Cuts"))
 (gr_line (start 159 117) (end 163 117) (stroke (width 0.05) (type default)) (layer "Edge.Cuts"))
 (gr_line (start 159 137) (end 151 137) (stroke (width 0.05) (type default)) (layer "Edge.Cuts"))
 (gr_line (start 159 142) (end 159 137) (stroke (width 0.05) (type default)) (layer "Edge.Cuts"))
 (gr_line (start 163 110) (end 159 110) (stroke (width 0.05) (type default)) (layer "Edge.Cuts"))
 (gr_line (start 163 110) (end 163 103) (stroke (width 0.05) (type default)) (layer "Edge.Cuts"))
 (gr_line (start 163 117) (end 163 126) (stroke (width 0.05) (type default)) (layer "Edge.Cuts"))
 (gr_line (start 163 126) (end 169 126) (stroke (width 0.05) (type default)) (layer "Edge.Cuts"))
 (gr_line (start 166 98) (end 166 103) (stroke (width 0.05) (type default)) (layer "Edge.Cuts"))
 (gr_line (start 166 103) (end 163 103) (stroke (width 0.05) (type default)) (layer "Edge.Cuts"))
 (gr_line (start 166 142) (end 159 142) (stroke (width 0.05) (type default)) (layer "Edge.Cuts"))
 (gr_line (start 166 146) (end 166 142) (stroke (width 0.05) (type default)) (layer "Edge.Cuts"))
 (gr_line (start 169 92) (end 169 98) (stroke (width 0.05) (type default)) (layer "Edge.Cuts"))
 (gr_line (start 169 98) (end 166 98) (stroke (width 0.05) (type default)) (layer "Edge.Cuts"))
 (gr_line (start 169 126) (end 169 132) (stroke (width 0.05) (type default)) (layer "Edge.Cuts"))
 (gr_line (start 169 132) (end 176 132) (stroke (width 0.05) (type default)) (layer "Edge.Cuts"))
 (gr_line (start 175 86) (end 175 92) (stroke (width 0.05) (type default)) (layer "Edge.Cuts"))
 (gr_line (start 175 92) (end 169 92) (stroke (width 0.05) (type default)) (layer "Edge.Cuts"))
 (gr_line (start 176 132) (end 176 137) (stroke (width 0.05) (type default)) (layer "Edge.Cuts"))
 (gr_line (start 176 137) (end 180 137) (stroke (width 0.05) (type default)) (layer "Edge.Cuts"))
 (gr_line (start 180 137) (end 180 146) (stroke (width 0.05) (type default)) (layer "Edge.Cuts"))
 (gr_line (start 180 146) (end 166 146) (stroke (width 0.05) (type default)) (layer "Edge.Cuts"))
 (gr_line (start 183 80) (end 183 86) (stroke (width 0.05) (type default)) (layer "Edge.Cuts"))
 (gr_line (start 183 86) (end 175 86) (stroke (width 0.05) (type default)) (layer "Edge.Cuts"))
 (segment (start 108.023654 118.65) (end 119.712654 118.65) (width 0.2) (layer "F.Cu") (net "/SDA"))
 (segment (start 106.95 109.56934) (end 106.95 117.576346) (width 0.2) (layer "F.Cu") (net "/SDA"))
 (segment (start 119.712654 118.65) (end 124.887654 123.825) (width 0.2) (layer "F.Cu") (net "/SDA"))
 (segment (start 119.275346 114.96) (end 126.514 122.198654) (width 0.2) (layer "F.Cu") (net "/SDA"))
 (segment (start 108.5 114.96) (end 119.275346 114.96) (width 0.2) (layer "F.Cu") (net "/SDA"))
 (segment (start 132.12 92.5) (end 132.12 91.125) (width 0.2) (layer "F.Cu") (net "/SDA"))
 (segment (start 124.887654 123.825) (end 125.840346 123.825) (width 0.2) (layer "F.Cu") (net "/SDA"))
 (segment (start 101.680101 87.34) (end 98.2 90.820101) (width 0.2) (layer "F.Cu") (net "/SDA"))
 (segment (start 126.514 122.198654) (end 126.514 123.151346) (width 0.2) (layer "F.Cu") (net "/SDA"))
 (segment (start 126.514 123.151346) (end 125.840346 123.825) (width 0.2) (layer "F.Cu") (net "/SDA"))
 (segment (start 98.2 100.81934) (end 106.95 109.56934) (width 0.2) (layer "F.Cu") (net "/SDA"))
 (segment (start 98.2 90.820101) (end 98.2 100.81934) (width 0.2) (layer "F.Cu") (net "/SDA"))
 (segment (start 106.95 117.576346) (end 108.023654 118.65) (width 0.2) (layer "F.Cu") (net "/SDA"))
 (segment (start 125.840346 123.825) (end 123.974 123.825) (width 0.2) (layer "F.Cu") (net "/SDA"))
 (segment (start 128.335 87.34) (end 101.680101 87.34) (width 0.2) (layer "F.Cu") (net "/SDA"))
 (segment (start 132.12 91.125) (end 128.335 87.34) (width 0.2) (layer "F.Cu") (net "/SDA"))
 (segment (start 123.974 123.825) (end 122.824 122.675) (width 0.2) (layer "F.Cu") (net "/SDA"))
 (segment (start 147.315 108.024899) (end 145.335101 110.004798) (width 0.2) (layer "F.Cu") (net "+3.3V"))
 (segment (start 99 92) (end 100 91) (width 0.2) (layer "F.Cu") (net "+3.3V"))
 (segment (start 145.335101 104.885202) (end 147.315 106.865101) (width 0.2) (layer "F.Cu") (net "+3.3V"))
 (segment (start 124.5 76.335) (end 145.335101 97.170101) (width 0.2) (layer "F.Cu") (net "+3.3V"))
 (segment (start 147.315 106.865101) (end 147.315 108.024899) (width 0.2) (layer "F.Cu") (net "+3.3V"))
 (segment (start 146.029899 124.4) (end 129.629 124.4) (width 0.2) (layer "F.Cu") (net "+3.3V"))
 (segment (start 107.9025 96.2125) (end 104.495 99.62) (width 0.2) (layer "F.Cu") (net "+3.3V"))
 (segment (start 99.585786 99.62) (end 99 99.034214) (width 0.2) (layer "F.Cu") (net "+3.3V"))
 (segment (start 147.315 123.114899) (end 146.029899 124.4) (width 0.2) (layer "F.Cu") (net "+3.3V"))
 (segment (start 127.904 116.214) (end 107.9025 96.2125) (width 0.2) (layer "F.Cu") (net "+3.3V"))
 (segment (start 145.335101 119.975202) (end 147.315 121.955101) (width 0.2) (layer "F.Cu") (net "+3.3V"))
 (segment (start 104.495 99.62) (end 99.585786 99.62) (width 0.2) (layer "F.Cu") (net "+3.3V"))
 (segment (start 99 99.034214) (end 99 92) (width 0.2) (layer "F.Cu") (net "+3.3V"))
 (segment (start 145.335101 110.004798) (end 145.335101 119.975202) (width 0.2) (layer "F.Cu") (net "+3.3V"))
 (segment (start 145.335101 97.170101) (end 145.335101 104.885202) (width 0.2) (layer "F.Cu") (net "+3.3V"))
 (segment (start 147.315 121.955101) (end 147.315 123.114899) (width 0.2) (layer "F.Cu") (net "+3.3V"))
 (segment (start 129.629 124.4) (end 127.904 122.675) (width 0.2) (layer "F.Cu") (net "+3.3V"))
 (segment (start 127.904 122.675) (end 127.904 116.214) (width 0.2) (layer "F.Cu") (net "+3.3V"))
 (segment (start 98.6 90.985786) (end 98.6 100.653654) (width 0.2) (layer "F.Cu") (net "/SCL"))
 (segment (start 99.585786 90) (end 98.6 90.985786) (width 0.2) (layer "F.Cu") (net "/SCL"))
 (segment (start 127.905 90.825) (end 123.661358 90.825) (width 0.2) (layer "F.Cu") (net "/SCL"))
 (segment (start 98.6 100.653654) (end 107.35 109.403654) (width 0.2) (layer "F.Cu") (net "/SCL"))
 (segment (start 123.661358 90.825) (end 122.836358 90) (width 0.2) (layer "F.Cu") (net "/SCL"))
 (segment (start 120.189 117.5) (end 125.364 122.675) (width 0.2) (layer "F.Cu") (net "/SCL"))
 (segment (start 107.35 109.403654) (end 107.35 116.35) (width 0.2) (layer "F.Cu") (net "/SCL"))
 (segment (start 108.5 117.5) (end 120.189 117.5) (width 0.2) (layer "F.Cu") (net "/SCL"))
 (segment (start 107.35 116.35) (end 108.5 117.5) (width 0.2) (layer "F.Cu") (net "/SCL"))
 (segment (start 122.836358 90) (end 99.585786 90) (width 0.2) (layer "F.Cu") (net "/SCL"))
 (segment (start 129.58 92.5) (end 127.905 90.825) (width 0.2) (layer "F.Cu") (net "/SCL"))
 (segment (start 108.405 94.175) (end 107.9025 93.6725) (width 0.2) (layer "F.Cu") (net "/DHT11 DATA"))
 (segment (start 107.9025 93.6725) (end 102.955 98.62) (width 0.2) (layer "F.Cu") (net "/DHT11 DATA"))
 (segment (start 120.285 94.175) (end 108.405 94.175) (width 0.2) (layer "F.Cu") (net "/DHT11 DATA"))
 (segment (start 102.955 98.62) (end 100 98.62) (width 0.2) (layer "F.Cu") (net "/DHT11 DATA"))
 (segment (start 121.96 92.5) (end 120.285 94.175) (width 0.2) (layer "F.Cu") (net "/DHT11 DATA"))
 (segment (start 124.5 103.5) (end 143.535 122.535) (width 0.2) (layer "F.Cu") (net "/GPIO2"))
 (segment (start 143.535 122.535) (end 145.915 122.535) (width 0.2) (layer "F.Cu") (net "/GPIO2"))
 (segment (start 124.5 92.5) (end 124.5 103.5) (width 0.2) (layer "F.Cu") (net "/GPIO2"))
 (segment (start 141.985 107.445) (end 145.915 107.445) (width 0.2) (layer "F.Cu") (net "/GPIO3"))
 (segment (start 127.04 92.5) (end 141.985 107.445) (width 0.2) (layer "F.Cu") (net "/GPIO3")))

